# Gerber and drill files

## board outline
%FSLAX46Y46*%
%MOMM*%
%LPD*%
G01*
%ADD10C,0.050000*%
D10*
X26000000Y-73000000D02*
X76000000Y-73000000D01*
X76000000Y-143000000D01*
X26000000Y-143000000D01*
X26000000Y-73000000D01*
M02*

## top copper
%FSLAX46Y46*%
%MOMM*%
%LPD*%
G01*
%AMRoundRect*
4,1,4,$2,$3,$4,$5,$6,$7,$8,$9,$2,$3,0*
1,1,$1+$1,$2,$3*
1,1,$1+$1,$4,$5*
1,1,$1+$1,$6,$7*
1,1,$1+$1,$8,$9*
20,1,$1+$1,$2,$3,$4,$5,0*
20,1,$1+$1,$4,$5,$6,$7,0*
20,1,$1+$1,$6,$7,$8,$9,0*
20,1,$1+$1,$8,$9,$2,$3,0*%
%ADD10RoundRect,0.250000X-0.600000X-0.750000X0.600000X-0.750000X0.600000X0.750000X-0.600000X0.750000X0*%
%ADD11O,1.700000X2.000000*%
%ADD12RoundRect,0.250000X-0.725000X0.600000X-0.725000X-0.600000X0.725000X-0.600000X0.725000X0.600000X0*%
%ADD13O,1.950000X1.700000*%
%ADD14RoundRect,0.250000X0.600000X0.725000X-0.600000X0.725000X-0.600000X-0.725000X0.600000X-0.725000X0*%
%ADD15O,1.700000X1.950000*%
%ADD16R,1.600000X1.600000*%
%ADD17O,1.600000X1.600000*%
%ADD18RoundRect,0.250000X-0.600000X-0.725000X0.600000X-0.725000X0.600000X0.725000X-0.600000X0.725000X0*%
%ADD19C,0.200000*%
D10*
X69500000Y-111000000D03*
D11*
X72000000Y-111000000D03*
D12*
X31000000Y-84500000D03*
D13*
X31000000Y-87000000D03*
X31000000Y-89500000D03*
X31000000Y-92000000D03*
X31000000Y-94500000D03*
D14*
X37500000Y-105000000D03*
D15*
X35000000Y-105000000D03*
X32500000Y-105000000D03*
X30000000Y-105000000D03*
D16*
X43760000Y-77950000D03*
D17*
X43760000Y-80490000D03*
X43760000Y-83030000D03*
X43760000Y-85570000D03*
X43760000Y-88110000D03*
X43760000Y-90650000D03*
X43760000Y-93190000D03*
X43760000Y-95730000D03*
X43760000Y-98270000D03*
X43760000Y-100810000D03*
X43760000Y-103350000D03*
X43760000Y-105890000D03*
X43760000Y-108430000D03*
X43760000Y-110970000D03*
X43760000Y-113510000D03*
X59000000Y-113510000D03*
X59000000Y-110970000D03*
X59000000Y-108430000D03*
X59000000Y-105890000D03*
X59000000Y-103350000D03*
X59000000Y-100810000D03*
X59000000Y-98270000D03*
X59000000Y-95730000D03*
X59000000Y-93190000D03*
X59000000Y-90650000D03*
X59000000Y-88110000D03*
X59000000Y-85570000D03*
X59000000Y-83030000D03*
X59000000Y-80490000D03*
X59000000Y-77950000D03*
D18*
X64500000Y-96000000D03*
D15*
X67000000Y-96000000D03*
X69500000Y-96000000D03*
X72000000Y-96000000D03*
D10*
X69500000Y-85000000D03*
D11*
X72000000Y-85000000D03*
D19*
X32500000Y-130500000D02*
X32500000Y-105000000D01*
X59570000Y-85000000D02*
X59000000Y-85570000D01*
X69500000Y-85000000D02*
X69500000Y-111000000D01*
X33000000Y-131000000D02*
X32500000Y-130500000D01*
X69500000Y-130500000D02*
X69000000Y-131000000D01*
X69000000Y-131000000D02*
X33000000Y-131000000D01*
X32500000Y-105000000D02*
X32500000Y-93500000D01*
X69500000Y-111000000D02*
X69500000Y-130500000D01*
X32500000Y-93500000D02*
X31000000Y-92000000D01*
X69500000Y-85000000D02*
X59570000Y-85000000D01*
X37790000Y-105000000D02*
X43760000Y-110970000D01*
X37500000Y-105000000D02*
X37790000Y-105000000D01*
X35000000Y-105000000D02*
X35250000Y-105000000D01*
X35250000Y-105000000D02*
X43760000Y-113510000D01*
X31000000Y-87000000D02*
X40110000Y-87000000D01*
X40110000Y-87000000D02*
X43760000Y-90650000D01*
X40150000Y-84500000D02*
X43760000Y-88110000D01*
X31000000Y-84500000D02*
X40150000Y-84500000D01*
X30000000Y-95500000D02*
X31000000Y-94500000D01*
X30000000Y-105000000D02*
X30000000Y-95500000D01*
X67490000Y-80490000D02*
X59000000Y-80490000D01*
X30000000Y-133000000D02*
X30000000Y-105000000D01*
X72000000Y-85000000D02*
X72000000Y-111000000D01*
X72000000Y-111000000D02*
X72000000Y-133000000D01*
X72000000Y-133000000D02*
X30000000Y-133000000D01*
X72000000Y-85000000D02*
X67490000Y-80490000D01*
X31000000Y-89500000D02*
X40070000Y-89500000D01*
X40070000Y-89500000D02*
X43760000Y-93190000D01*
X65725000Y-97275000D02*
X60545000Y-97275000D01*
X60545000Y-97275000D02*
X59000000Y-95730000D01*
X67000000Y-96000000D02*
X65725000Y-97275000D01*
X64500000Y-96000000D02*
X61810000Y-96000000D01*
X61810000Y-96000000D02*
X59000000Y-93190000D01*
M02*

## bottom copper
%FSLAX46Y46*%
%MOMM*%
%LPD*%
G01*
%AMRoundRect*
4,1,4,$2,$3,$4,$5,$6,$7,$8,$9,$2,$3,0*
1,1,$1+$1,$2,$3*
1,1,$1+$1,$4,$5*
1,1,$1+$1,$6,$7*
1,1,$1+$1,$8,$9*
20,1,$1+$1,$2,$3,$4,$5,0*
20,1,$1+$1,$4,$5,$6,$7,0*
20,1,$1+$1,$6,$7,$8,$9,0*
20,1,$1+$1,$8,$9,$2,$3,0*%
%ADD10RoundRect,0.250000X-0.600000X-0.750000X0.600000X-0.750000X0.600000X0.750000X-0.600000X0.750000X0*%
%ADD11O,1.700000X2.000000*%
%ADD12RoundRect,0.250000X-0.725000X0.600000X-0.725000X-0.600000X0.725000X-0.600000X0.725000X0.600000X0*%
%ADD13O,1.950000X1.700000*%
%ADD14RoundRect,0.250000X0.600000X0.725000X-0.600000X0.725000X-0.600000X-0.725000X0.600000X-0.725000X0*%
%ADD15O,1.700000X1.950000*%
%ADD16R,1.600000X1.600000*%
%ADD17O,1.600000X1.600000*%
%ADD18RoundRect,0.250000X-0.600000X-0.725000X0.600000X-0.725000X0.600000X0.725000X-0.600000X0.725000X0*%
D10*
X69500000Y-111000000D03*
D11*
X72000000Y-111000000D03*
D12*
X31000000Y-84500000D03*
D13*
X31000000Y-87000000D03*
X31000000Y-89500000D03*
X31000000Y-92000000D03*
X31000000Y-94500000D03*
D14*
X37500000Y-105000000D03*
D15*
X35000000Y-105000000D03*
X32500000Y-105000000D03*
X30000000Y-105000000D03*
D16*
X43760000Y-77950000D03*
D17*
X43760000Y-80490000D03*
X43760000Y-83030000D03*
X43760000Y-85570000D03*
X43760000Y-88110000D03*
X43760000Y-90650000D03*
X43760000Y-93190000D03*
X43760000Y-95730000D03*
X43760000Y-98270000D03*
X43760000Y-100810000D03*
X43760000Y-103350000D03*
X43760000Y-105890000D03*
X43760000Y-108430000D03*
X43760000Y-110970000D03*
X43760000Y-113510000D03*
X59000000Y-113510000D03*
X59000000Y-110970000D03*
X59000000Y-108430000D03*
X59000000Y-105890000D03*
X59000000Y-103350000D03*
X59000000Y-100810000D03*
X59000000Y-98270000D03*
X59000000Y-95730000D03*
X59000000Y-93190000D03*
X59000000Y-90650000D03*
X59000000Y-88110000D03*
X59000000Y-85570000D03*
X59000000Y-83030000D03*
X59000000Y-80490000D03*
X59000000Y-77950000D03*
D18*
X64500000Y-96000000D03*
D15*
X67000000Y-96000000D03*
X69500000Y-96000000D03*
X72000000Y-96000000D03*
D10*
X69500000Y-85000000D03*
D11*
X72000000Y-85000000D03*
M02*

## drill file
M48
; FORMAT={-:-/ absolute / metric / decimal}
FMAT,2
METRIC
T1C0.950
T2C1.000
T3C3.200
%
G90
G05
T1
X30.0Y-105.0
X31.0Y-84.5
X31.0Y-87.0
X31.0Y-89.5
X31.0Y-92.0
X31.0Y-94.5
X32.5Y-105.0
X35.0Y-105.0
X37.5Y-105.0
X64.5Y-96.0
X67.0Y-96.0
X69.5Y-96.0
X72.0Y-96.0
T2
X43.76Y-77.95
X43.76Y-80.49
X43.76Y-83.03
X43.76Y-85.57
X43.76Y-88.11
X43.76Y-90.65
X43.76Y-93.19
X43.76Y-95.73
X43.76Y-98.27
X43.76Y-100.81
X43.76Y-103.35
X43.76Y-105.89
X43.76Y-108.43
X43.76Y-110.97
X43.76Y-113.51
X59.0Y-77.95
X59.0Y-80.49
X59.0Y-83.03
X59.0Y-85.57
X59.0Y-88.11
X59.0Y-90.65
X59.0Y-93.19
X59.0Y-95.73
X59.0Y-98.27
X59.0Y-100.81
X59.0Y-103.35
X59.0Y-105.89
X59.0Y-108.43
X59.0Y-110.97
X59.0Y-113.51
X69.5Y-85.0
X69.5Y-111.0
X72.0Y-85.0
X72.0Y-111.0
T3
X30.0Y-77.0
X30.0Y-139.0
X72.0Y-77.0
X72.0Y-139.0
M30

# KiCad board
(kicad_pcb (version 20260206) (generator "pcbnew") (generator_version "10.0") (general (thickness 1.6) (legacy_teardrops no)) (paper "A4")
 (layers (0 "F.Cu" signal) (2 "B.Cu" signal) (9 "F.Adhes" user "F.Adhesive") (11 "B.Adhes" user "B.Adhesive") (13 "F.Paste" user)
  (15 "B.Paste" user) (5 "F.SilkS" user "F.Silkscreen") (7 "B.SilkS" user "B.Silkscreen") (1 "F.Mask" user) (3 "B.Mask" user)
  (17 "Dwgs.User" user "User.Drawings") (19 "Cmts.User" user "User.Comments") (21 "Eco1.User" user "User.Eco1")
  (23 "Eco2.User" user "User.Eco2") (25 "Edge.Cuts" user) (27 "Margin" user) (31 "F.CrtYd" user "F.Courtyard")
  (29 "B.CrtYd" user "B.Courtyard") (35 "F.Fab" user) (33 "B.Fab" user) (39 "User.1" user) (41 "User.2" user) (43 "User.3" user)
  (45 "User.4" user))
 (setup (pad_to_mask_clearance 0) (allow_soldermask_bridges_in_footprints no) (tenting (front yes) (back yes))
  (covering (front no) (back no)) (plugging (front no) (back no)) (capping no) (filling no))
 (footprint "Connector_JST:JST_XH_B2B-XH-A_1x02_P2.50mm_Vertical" (layer "F.Cu") (at 69.5 111)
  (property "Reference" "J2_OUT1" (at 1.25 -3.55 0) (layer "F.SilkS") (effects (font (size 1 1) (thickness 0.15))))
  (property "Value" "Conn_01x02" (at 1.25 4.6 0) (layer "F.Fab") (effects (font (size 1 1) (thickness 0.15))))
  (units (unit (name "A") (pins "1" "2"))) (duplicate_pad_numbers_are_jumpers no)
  (pad "1" thru_hole roundrect (at 0 0) (size 1.7 2) (drill 1) (layers "*.Cu" "*.Mask") (remove_unused_layers no)
   (roundrect_rratio 0.147059) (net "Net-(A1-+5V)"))
  (pad "2" thru_hole oval (at 2.5 0) (size 1.7 2) (drill 1) (layers "*.Cu" "*.Mask") (remove_unused_layers no) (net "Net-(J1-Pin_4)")))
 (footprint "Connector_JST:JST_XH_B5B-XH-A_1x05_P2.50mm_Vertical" (layer "F.Cu") (at 31 84.5 -90)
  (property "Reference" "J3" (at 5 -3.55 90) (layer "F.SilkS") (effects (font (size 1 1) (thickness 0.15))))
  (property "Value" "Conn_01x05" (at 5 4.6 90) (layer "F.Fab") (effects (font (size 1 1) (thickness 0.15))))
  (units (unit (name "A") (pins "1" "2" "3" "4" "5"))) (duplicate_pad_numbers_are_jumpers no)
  (pad "1" thru_hole roundrect (at 0 0 270) (size 1.7 1.95) (drill 0.95) (layers "*.Cu" "*.Mask") (remove_unused_layers no)
   (roundrect_rratio 0.147059) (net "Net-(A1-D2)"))
  (pad "2" thru_hole oval (at 2.5 0 270) (size 1.7 1.95) (drill 0.95) (layers "*.Cu" "*.Mask") (remove_unused_layers no) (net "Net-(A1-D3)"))
  (pad "3" thru_hole oval (at 5 0 270) (size 1.7 1.95) (drill 0.95) (layers "*.Cu" "*.Mask") (remove_unused_layers no) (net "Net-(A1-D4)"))
  (pad "4" thru_hole oval (at 7.5 0 270) (size 1.7 1.95) (drill 0.95) (layers "*.Cu" "*.Mask") (remove_unused_layers no)
   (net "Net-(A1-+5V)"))
  (pad "5" thru_hole oval (at 10 0 270) (size 1.7 1.95) (drill 0.95) (layers "*.Cu" "*.Mask") (remove_unused_layers no)
   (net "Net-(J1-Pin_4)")))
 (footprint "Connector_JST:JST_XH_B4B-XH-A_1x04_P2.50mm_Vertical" (layer "F.Cu") (at 37.5 105 180)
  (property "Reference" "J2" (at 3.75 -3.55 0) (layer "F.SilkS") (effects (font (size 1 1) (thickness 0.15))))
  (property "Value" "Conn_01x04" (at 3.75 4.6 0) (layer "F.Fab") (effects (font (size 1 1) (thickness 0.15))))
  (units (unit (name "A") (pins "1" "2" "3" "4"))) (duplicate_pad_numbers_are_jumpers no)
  (pad "1" thru_hole roundrect (at 0 0 180) (size 1.7 1.95) (drill 0.95) (layers "*.Cu" "*.Mask") (remove_unused_layers no)
   (roundrect_rratio 0.147059) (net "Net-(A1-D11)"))
  (pad "2" thru_hole oval (at 2.5 0 180) (size 1.7 1.95) (drill 0.95) (layers "*.Cu" "*.Mask") (remove_unused_layers no)
   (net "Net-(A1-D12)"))
  (pad "3" thru_hole oval (at 5 0 180) (size 1.7 1.95) (drill 0.95) (layers "*.Cu" "*.Mask") (remove_unused_layers no) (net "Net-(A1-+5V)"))
  (pad "4" thru_hole oval (at 7.5 0 180) (size 1.7 1.95) (drill 0.95) (layers "*.Cu" "*.Mask") (remove_unused_layers no)
   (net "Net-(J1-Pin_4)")))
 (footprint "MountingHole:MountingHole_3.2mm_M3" (layer "F.Cu") (at 72 139)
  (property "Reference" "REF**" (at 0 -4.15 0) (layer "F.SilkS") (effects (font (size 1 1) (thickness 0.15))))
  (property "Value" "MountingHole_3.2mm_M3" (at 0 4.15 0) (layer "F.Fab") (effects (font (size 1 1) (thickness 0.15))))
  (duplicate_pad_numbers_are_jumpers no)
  (pad "" np_thru_hole circle (at 0 0) (size 3.2 3.2) (drill 3.2) (layers "*.Cu" "*.Mask")))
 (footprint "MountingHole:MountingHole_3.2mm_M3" (layer "F.Cu") (at 30 139)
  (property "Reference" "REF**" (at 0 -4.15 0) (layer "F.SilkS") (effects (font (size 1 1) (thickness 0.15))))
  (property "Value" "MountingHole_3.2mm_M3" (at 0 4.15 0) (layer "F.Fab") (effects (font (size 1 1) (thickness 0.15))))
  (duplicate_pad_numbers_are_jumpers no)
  (pad "" np_thru_hole circle (at 0 0) (size 3.2 3.2) (drill 3.2) (layers "*.Cu" "*.Mask")))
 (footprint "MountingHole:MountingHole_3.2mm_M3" (layer "F.Cu") (at 30 77)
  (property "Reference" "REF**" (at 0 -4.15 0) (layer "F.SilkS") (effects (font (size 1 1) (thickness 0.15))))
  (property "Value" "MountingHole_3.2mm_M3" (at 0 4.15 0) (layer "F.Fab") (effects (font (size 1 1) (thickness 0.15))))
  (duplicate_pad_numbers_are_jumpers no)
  (pad "" np_thru_hole circle (at 0 0) (size 3.2 3.2) (drill 3.2) (layers "*.Cu" "*.Mask")))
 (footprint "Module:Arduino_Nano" (layer "F.Cu") (at 43.76 77.95)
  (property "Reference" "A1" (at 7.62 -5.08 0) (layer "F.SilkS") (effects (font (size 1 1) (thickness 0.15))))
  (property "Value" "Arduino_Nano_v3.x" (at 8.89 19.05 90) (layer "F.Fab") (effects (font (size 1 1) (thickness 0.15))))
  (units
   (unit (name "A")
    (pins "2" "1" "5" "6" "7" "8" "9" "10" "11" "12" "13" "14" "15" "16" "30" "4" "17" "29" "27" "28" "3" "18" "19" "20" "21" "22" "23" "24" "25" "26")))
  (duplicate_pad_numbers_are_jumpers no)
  (pad "1" thru_hole rect (at 0 0) (size 1.6 1.6) (drill 1) (layers "*.Cu" "*.Mask") (remove_unused_layers no)
   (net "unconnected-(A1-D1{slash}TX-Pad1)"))
  (pad "2" thru_hole oval (at 0 2.54) (size 1.6 1.6) (drill 1) (layers "*.Cu" "*.Mask") (remove_unused_layers no)
   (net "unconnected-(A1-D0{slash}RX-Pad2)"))
  (pad "3" thru_hole oval (at 0 5.08) (size 1.6 1.6) (drill 1) (layers "*.Cu" "*.Mask") (remove_unused_layers no)
   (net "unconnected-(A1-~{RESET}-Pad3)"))
  (pad "4" thru_hole oval (at 0 7.62) (size 1.6 1.6) (drill 1) (layers "*.Cu" "*.Mask") (remove_unused_layers no)
   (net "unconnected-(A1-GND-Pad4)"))
  (pad "5" thru_hole oval (at 0 10.16) (size 1.6 1.6) (drill 1) (layers "*.Cu" "*.Mask") (remove_unused_layers no) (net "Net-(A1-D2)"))
  (pad "6" thru_hole oval (at 0 12.7) (size 1.6 1.6) (drill 1) (layers "*.Cu" "*.Mask") (remove_unused_layers no) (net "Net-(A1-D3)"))
  (pad "7" thru_hole oval (at 0 15.24) (size 1.6 1.6) (drill 1) (layers "*.Cu" "*.Mask") (remove_unused_layers no) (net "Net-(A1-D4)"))
  (pad "8" thru_hole oval (at 0 17.78) (size 1.6 1.6) (drill 1) (layers "*.Cu" "*.Mask") (remove_unused_layers no)
   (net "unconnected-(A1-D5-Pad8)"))
  (pad "9" thru_hole oval (at 0 20.32) (size 1.6 1.6) (drill 1) (layers "*.Cu" "*.Mask") (remove_unused_layers no)
   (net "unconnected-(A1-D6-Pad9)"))
  (pad "10" thru_hole oval (at 0 22.86) (size 1.6 1.6) (drill 1) (layers "*.Cu" "*.Mask") (remove_unused_layers no)
   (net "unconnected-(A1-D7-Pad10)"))
  (pad "11" thru_hole oval (at 0 25.4) (size 1.6 1.6) (drill 1) (layers "*.Cu" "*.Mask") (remove_unused_layers no)
   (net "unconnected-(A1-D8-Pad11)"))
  (pad "12" thru_hole oval (at 0 27.94) (size 1.6 1.6) (drill 1) (layers "*.Cu" "*.Mask") (remove_unused_layers no)
   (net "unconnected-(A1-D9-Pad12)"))
  (pad "13" thru_hole oval (at 0 30.48) (size 1.6 1.6) (drill 1) (layers "*.Cu" "*.Mask") (remove_unused_layers no)
   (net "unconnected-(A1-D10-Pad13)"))
  (pad "14" thru_hole oval (at 0 33.02) (size 1.6 1.6) (drill 1) (layers "*.Cu" "*.Mask") (remove_unused_layers no) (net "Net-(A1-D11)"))
  (pad "15" thru_hole oval (at 0 35.56) (size 1.6 1.6) (drill 1) (layers "*.Cu" "*.Mask") (remove_unused_layers no) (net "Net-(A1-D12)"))
  (pad "16" thru_hole oval (at 15.24 35.56) (size 1.6 1.6) (drill 1) (layers "*.Cu" "*.Mask") (remove_unused_layers no)
   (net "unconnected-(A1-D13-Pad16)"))
  (pad "17" thru_hole oval (at 15.24 33.02) (size 1.6 1.6) (drill 1) (layers "*.Cu" "*.Mask") (remove_unused_layers no)
   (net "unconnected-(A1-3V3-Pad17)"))
  (pad "18" thru_hole oval (at 15.24 30.48) (size 1.6 1.6) (drill 1) (layers "*.Cu" "*.Mask") (remove_unused_layers no)
   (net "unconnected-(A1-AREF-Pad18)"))
  (pad "19" thru_hole oval (at 15.24 27.94) (size 1.6 1.6) (drill 1) (layers "*.Cu" "*.Mask") (remove_unused_layers no)
   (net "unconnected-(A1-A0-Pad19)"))
  (pad "20" thru_hole oval (at 15.24 25.4) (size 1.6 1.6) (drill 1) (layers "*.Cu" "*.Mask") (remove_unused_layers no)
   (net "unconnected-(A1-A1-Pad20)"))
  (pad "21" thru_hole oval (at 15.24 22.86) (size 1.6 1.6) (drill 1) (layers "*.Cu" "*.Mask") (remove_unused_layers no)
   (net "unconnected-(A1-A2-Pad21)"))
  (pad "22" thru_hole oval (at 15.24 20.32) (size 1.6 1.6) (drill 1) (layers "*.Cu" "*.Mask") (remove_unused_layers no)
   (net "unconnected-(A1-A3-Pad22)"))
  (pad "23" thru_hole oval (at 15.24 17.78) (size 1.6 1.6) (drill 1) (layers "*.Cu" "*.Mask") (remove_unused_layers no) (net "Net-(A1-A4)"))
  (pad "24" thru_hole oval (at 15.24 15.24) (size 1.6 1.6) (drill 1) (layers "*.Cu" "*.Mask") (remove_unused_layers no) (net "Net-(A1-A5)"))
  (pad "25" thru_hole oval (at 15.24 12.7) (size 1.6 1.6) (drill 1) (layers "*.Cu" "*.Mask") (remove_unused_layers no)
   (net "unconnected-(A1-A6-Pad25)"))
  (pad "26" thru_hole oval (at 15.24 10.16) (size 1.6 1.6) (drill 1) (layers "*.Cu" "*.Mask") (remove_unused_layers no)
   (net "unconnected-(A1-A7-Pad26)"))
  (pad "27" thru_hole oval (at 15.24 7.62) (size 1.6 1.6) (drill 1) (layers "*.Cu" "*.Mask") (remove_unused_layers no) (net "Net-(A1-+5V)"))
  (pad "28" thru_hole oval (at 15.24 5.08) (size 1.6 1.6) (drill 1) (layers "*.Cu" "*.Mask") (remove_unused_layers no)
   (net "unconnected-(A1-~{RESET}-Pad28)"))
  (pad "29" thru_hole oval (at 15.24 2.54) (size 1.6 1.6) (drill 1) (layers "*.Cu" "*.Mask") (remove_unused_layers no)
   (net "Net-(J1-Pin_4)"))
  (pad "30" thru_hole oval (at 15.24 0) (size 1.6 1.6) (drill 1) (layers "*.Cu" "*.Mask") (remove_unused_layers no)
   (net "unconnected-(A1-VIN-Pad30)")))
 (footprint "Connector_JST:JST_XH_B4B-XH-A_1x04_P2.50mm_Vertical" (layer "F.Cu") (at 64.5 96)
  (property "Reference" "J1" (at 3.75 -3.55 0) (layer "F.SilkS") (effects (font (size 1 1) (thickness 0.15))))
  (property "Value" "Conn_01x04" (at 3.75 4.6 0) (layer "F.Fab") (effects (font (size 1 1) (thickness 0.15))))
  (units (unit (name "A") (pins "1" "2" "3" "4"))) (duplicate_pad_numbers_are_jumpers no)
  (pad "1" thru_hole roundrect (at 0 0) (size 1.7 1.95) (drill 0.95) (layers "*.Cu" "*.Mask") (remove_unused_layers no)
   (roundrect_rratio 0.147059) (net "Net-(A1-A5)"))
  (pad "2" thru_hole oval (at 2.5 0) (size 1.7 1.95) (drill 0.95) (layers "*.Cu" "*.Mask") (remove_unused_layers no) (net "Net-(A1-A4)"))
  (pad "3" thru_hole oval (at 5 0) (size 1.7 1.95) (drill 0.95) (layers "*.Cu" "*.Mask") (remove_unused_layers no) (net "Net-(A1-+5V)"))
  (pad "4" thru_hole oval (at 7.5 0) (size 1.7 1.95) (drill 0.95) (layers "*.Cu" "*.Mask") (remove_unused_layers no) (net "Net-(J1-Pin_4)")))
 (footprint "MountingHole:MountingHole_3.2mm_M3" (layer "F.Cu") (at 72 77)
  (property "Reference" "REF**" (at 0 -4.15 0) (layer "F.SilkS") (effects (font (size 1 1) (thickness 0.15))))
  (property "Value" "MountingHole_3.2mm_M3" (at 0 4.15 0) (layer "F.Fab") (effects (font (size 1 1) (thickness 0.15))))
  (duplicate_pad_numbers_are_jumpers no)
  (pad "" np_thru_hole circle (at 0 0) (size 3.2 3.2) (drill 3.2) (layers "*.Cu" "*.Mask")))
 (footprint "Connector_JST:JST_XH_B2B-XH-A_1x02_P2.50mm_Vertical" (layer "F.Cu") (at 69.5 85)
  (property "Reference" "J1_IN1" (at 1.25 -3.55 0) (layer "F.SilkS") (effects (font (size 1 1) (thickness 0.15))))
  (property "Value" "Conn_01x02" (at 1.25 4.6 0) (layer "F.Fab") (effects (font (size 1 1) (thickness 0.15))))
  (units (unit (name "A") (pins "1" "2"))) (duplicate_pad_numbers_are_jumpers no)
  (pad "1" thru_hole roundrect (at 0 0) (size 1.7 2) (drill 1) (layers "*.Cu" "*.Mask") (remove_unused_layers no)
   (roundrect_rratio 0.147059) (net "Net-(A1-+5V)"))
  (pad "2" thru_hole oval (at 2.5 0) (size 1.7 2) (drill 1) (layers "*.Cu" "*.Mask") (remove_unused_layers no) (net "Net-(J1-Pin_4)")))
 (gr_rect (start 26 73) (end 76 143) (stroke (width 0.05) (type default)) (fill no) (layer "Edge.Cuts"))
 (segment (start 32.5 130.5) (end 32.5 105) (width 0.2) (layer "F.Cu") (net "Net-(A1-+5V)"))
 (segment (start 59.57 85) (end 59 85.57) (width 0.2) (layer "F.Cu") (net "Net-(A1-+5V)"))
 (segment (start 69.5 85) (end 69.5 111) (width 0.2) (layer "F.Cu") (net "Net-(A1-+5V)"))
 (segment (start 33 131) (end 32.5 130.5) (width 0.2) (layer "F.Cu") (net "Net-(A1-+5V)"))
 (segment (start 69.5 130.5) (end 69 131) (width 0.2) (layer "F.Cu") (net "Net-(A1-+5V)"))
 (segment (start 69 131) (end 33 131) (width 0.2) (layer "F.Cu") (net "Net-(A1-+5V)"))
 (segment (start 32.5 105) (end 32.5 93.5) (width 0.2) (layer "F.Cu") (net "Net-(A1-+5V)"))
 (segment (start 69.5 111) (end 69.5 130.5) (width 0.2) (layer "F.Cu") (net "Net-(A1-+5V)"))
 (segment (start 32.5 93.5) (end 31 92) (width 0.2) (layer "F.Cu") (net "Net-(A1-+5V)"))
 (segment (start 69.5 85) (end 59.57 85) (width 0.2) (layer "F.Cu") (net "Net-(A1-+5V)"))
 (segment (start 37.79 105) (end 43.76 110.97) (width 0.2) (layer "F.Cu") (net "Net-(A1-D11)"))
 (segment (start 37.5 105) (end 37.79 105) (width 0.2) (layer "F.Cu") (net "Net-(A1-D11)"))
 (segment (start 35 105) (end 35.25 105) (width 0.2) (layer "F.Cu") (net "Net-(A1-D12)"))
 (segment (start 35.25 105) (end 43.76 113.51) (width 0.2) (layer "F.Cu") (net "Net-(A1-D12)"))
 (segment (start 31 87) (end 40.11 87) (width 0.2) (layer "F.Cu") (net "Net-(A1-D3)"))
 (segment (start 40.11 87) (end 43.76 90.65) (width 0.2) (layer "F.Cu") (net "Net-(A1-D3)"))
 (segment (start 40.15 84.5) (end 43.76 88.11) (width 0.2) (layer "F.Cu") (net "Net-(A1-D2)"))
 (segment (start 31 84.5) (end 40.15 84.5) (width 0.2) (layer "F.Cu") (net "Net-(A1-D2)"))
 (segment (start 30 95.5) (end 31 94.5) (width 0.2) (layer "F.Cu") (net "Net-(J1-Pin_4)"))
 (segment (start 30 105) (end 30 95.5) (width 0.2) (layer "F.Cu") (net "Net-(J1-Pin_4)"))
 (segment (start 67.49 80.49) (end 59 80.49) (width 0.2) (layer "F.Cu") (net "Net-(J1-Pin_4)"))
 (segment (start 30 133) (end 30 105) (width 0.2) (layer "F.Cu") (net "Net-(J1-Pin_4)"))
 (segment (start 72 85) (end 72 111) (width 0.2) (layer "F.Cu") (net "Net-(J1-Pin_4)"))
 (segment (start 72 111) (end 72 133) (width 0.2) (layer "F.Cu") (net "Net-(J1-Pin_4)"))
 (segment (start 72 133) (end 30 133) (width 0.2) (layer "F.Cu") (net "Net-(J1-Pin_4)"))
 (segment (start 72 85) (end 67.49 80.49) (width 0.2) (layer "F.Cu") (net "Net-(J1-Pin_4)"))
 (segment (start 31 89.5) (end 40.07 89.5) (width 0.2) (layer "F.Cu") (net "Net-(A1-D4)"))
 (segment (start 40.07 89.5) (end 43.76 93.19) (width 0.2) (layer "F.Cu") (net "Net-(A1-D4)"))
 (segment (start 65.725 97.275) (end 60.545 97.275) (width 0.2) (layer "F.Cu") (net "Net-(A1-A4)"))
 (segment (start 60.545 97.275) (end 59 95.73) (width 0.2) (layer "F.Cu") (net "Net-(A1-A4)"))
 (segment (start 67 96) (end 65.725 97.275) (width 0.2) (layer "F.Cu") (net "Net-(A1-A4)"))
 (segment (start 64.5 96) (end 61.81 96) (width 0.2) (layer "F.Cu") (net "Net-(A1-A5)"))
 (segment (start 61.81 96) (end 59 93.19) (width 0.2) (layer "F.Cu") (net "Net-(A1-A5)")))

